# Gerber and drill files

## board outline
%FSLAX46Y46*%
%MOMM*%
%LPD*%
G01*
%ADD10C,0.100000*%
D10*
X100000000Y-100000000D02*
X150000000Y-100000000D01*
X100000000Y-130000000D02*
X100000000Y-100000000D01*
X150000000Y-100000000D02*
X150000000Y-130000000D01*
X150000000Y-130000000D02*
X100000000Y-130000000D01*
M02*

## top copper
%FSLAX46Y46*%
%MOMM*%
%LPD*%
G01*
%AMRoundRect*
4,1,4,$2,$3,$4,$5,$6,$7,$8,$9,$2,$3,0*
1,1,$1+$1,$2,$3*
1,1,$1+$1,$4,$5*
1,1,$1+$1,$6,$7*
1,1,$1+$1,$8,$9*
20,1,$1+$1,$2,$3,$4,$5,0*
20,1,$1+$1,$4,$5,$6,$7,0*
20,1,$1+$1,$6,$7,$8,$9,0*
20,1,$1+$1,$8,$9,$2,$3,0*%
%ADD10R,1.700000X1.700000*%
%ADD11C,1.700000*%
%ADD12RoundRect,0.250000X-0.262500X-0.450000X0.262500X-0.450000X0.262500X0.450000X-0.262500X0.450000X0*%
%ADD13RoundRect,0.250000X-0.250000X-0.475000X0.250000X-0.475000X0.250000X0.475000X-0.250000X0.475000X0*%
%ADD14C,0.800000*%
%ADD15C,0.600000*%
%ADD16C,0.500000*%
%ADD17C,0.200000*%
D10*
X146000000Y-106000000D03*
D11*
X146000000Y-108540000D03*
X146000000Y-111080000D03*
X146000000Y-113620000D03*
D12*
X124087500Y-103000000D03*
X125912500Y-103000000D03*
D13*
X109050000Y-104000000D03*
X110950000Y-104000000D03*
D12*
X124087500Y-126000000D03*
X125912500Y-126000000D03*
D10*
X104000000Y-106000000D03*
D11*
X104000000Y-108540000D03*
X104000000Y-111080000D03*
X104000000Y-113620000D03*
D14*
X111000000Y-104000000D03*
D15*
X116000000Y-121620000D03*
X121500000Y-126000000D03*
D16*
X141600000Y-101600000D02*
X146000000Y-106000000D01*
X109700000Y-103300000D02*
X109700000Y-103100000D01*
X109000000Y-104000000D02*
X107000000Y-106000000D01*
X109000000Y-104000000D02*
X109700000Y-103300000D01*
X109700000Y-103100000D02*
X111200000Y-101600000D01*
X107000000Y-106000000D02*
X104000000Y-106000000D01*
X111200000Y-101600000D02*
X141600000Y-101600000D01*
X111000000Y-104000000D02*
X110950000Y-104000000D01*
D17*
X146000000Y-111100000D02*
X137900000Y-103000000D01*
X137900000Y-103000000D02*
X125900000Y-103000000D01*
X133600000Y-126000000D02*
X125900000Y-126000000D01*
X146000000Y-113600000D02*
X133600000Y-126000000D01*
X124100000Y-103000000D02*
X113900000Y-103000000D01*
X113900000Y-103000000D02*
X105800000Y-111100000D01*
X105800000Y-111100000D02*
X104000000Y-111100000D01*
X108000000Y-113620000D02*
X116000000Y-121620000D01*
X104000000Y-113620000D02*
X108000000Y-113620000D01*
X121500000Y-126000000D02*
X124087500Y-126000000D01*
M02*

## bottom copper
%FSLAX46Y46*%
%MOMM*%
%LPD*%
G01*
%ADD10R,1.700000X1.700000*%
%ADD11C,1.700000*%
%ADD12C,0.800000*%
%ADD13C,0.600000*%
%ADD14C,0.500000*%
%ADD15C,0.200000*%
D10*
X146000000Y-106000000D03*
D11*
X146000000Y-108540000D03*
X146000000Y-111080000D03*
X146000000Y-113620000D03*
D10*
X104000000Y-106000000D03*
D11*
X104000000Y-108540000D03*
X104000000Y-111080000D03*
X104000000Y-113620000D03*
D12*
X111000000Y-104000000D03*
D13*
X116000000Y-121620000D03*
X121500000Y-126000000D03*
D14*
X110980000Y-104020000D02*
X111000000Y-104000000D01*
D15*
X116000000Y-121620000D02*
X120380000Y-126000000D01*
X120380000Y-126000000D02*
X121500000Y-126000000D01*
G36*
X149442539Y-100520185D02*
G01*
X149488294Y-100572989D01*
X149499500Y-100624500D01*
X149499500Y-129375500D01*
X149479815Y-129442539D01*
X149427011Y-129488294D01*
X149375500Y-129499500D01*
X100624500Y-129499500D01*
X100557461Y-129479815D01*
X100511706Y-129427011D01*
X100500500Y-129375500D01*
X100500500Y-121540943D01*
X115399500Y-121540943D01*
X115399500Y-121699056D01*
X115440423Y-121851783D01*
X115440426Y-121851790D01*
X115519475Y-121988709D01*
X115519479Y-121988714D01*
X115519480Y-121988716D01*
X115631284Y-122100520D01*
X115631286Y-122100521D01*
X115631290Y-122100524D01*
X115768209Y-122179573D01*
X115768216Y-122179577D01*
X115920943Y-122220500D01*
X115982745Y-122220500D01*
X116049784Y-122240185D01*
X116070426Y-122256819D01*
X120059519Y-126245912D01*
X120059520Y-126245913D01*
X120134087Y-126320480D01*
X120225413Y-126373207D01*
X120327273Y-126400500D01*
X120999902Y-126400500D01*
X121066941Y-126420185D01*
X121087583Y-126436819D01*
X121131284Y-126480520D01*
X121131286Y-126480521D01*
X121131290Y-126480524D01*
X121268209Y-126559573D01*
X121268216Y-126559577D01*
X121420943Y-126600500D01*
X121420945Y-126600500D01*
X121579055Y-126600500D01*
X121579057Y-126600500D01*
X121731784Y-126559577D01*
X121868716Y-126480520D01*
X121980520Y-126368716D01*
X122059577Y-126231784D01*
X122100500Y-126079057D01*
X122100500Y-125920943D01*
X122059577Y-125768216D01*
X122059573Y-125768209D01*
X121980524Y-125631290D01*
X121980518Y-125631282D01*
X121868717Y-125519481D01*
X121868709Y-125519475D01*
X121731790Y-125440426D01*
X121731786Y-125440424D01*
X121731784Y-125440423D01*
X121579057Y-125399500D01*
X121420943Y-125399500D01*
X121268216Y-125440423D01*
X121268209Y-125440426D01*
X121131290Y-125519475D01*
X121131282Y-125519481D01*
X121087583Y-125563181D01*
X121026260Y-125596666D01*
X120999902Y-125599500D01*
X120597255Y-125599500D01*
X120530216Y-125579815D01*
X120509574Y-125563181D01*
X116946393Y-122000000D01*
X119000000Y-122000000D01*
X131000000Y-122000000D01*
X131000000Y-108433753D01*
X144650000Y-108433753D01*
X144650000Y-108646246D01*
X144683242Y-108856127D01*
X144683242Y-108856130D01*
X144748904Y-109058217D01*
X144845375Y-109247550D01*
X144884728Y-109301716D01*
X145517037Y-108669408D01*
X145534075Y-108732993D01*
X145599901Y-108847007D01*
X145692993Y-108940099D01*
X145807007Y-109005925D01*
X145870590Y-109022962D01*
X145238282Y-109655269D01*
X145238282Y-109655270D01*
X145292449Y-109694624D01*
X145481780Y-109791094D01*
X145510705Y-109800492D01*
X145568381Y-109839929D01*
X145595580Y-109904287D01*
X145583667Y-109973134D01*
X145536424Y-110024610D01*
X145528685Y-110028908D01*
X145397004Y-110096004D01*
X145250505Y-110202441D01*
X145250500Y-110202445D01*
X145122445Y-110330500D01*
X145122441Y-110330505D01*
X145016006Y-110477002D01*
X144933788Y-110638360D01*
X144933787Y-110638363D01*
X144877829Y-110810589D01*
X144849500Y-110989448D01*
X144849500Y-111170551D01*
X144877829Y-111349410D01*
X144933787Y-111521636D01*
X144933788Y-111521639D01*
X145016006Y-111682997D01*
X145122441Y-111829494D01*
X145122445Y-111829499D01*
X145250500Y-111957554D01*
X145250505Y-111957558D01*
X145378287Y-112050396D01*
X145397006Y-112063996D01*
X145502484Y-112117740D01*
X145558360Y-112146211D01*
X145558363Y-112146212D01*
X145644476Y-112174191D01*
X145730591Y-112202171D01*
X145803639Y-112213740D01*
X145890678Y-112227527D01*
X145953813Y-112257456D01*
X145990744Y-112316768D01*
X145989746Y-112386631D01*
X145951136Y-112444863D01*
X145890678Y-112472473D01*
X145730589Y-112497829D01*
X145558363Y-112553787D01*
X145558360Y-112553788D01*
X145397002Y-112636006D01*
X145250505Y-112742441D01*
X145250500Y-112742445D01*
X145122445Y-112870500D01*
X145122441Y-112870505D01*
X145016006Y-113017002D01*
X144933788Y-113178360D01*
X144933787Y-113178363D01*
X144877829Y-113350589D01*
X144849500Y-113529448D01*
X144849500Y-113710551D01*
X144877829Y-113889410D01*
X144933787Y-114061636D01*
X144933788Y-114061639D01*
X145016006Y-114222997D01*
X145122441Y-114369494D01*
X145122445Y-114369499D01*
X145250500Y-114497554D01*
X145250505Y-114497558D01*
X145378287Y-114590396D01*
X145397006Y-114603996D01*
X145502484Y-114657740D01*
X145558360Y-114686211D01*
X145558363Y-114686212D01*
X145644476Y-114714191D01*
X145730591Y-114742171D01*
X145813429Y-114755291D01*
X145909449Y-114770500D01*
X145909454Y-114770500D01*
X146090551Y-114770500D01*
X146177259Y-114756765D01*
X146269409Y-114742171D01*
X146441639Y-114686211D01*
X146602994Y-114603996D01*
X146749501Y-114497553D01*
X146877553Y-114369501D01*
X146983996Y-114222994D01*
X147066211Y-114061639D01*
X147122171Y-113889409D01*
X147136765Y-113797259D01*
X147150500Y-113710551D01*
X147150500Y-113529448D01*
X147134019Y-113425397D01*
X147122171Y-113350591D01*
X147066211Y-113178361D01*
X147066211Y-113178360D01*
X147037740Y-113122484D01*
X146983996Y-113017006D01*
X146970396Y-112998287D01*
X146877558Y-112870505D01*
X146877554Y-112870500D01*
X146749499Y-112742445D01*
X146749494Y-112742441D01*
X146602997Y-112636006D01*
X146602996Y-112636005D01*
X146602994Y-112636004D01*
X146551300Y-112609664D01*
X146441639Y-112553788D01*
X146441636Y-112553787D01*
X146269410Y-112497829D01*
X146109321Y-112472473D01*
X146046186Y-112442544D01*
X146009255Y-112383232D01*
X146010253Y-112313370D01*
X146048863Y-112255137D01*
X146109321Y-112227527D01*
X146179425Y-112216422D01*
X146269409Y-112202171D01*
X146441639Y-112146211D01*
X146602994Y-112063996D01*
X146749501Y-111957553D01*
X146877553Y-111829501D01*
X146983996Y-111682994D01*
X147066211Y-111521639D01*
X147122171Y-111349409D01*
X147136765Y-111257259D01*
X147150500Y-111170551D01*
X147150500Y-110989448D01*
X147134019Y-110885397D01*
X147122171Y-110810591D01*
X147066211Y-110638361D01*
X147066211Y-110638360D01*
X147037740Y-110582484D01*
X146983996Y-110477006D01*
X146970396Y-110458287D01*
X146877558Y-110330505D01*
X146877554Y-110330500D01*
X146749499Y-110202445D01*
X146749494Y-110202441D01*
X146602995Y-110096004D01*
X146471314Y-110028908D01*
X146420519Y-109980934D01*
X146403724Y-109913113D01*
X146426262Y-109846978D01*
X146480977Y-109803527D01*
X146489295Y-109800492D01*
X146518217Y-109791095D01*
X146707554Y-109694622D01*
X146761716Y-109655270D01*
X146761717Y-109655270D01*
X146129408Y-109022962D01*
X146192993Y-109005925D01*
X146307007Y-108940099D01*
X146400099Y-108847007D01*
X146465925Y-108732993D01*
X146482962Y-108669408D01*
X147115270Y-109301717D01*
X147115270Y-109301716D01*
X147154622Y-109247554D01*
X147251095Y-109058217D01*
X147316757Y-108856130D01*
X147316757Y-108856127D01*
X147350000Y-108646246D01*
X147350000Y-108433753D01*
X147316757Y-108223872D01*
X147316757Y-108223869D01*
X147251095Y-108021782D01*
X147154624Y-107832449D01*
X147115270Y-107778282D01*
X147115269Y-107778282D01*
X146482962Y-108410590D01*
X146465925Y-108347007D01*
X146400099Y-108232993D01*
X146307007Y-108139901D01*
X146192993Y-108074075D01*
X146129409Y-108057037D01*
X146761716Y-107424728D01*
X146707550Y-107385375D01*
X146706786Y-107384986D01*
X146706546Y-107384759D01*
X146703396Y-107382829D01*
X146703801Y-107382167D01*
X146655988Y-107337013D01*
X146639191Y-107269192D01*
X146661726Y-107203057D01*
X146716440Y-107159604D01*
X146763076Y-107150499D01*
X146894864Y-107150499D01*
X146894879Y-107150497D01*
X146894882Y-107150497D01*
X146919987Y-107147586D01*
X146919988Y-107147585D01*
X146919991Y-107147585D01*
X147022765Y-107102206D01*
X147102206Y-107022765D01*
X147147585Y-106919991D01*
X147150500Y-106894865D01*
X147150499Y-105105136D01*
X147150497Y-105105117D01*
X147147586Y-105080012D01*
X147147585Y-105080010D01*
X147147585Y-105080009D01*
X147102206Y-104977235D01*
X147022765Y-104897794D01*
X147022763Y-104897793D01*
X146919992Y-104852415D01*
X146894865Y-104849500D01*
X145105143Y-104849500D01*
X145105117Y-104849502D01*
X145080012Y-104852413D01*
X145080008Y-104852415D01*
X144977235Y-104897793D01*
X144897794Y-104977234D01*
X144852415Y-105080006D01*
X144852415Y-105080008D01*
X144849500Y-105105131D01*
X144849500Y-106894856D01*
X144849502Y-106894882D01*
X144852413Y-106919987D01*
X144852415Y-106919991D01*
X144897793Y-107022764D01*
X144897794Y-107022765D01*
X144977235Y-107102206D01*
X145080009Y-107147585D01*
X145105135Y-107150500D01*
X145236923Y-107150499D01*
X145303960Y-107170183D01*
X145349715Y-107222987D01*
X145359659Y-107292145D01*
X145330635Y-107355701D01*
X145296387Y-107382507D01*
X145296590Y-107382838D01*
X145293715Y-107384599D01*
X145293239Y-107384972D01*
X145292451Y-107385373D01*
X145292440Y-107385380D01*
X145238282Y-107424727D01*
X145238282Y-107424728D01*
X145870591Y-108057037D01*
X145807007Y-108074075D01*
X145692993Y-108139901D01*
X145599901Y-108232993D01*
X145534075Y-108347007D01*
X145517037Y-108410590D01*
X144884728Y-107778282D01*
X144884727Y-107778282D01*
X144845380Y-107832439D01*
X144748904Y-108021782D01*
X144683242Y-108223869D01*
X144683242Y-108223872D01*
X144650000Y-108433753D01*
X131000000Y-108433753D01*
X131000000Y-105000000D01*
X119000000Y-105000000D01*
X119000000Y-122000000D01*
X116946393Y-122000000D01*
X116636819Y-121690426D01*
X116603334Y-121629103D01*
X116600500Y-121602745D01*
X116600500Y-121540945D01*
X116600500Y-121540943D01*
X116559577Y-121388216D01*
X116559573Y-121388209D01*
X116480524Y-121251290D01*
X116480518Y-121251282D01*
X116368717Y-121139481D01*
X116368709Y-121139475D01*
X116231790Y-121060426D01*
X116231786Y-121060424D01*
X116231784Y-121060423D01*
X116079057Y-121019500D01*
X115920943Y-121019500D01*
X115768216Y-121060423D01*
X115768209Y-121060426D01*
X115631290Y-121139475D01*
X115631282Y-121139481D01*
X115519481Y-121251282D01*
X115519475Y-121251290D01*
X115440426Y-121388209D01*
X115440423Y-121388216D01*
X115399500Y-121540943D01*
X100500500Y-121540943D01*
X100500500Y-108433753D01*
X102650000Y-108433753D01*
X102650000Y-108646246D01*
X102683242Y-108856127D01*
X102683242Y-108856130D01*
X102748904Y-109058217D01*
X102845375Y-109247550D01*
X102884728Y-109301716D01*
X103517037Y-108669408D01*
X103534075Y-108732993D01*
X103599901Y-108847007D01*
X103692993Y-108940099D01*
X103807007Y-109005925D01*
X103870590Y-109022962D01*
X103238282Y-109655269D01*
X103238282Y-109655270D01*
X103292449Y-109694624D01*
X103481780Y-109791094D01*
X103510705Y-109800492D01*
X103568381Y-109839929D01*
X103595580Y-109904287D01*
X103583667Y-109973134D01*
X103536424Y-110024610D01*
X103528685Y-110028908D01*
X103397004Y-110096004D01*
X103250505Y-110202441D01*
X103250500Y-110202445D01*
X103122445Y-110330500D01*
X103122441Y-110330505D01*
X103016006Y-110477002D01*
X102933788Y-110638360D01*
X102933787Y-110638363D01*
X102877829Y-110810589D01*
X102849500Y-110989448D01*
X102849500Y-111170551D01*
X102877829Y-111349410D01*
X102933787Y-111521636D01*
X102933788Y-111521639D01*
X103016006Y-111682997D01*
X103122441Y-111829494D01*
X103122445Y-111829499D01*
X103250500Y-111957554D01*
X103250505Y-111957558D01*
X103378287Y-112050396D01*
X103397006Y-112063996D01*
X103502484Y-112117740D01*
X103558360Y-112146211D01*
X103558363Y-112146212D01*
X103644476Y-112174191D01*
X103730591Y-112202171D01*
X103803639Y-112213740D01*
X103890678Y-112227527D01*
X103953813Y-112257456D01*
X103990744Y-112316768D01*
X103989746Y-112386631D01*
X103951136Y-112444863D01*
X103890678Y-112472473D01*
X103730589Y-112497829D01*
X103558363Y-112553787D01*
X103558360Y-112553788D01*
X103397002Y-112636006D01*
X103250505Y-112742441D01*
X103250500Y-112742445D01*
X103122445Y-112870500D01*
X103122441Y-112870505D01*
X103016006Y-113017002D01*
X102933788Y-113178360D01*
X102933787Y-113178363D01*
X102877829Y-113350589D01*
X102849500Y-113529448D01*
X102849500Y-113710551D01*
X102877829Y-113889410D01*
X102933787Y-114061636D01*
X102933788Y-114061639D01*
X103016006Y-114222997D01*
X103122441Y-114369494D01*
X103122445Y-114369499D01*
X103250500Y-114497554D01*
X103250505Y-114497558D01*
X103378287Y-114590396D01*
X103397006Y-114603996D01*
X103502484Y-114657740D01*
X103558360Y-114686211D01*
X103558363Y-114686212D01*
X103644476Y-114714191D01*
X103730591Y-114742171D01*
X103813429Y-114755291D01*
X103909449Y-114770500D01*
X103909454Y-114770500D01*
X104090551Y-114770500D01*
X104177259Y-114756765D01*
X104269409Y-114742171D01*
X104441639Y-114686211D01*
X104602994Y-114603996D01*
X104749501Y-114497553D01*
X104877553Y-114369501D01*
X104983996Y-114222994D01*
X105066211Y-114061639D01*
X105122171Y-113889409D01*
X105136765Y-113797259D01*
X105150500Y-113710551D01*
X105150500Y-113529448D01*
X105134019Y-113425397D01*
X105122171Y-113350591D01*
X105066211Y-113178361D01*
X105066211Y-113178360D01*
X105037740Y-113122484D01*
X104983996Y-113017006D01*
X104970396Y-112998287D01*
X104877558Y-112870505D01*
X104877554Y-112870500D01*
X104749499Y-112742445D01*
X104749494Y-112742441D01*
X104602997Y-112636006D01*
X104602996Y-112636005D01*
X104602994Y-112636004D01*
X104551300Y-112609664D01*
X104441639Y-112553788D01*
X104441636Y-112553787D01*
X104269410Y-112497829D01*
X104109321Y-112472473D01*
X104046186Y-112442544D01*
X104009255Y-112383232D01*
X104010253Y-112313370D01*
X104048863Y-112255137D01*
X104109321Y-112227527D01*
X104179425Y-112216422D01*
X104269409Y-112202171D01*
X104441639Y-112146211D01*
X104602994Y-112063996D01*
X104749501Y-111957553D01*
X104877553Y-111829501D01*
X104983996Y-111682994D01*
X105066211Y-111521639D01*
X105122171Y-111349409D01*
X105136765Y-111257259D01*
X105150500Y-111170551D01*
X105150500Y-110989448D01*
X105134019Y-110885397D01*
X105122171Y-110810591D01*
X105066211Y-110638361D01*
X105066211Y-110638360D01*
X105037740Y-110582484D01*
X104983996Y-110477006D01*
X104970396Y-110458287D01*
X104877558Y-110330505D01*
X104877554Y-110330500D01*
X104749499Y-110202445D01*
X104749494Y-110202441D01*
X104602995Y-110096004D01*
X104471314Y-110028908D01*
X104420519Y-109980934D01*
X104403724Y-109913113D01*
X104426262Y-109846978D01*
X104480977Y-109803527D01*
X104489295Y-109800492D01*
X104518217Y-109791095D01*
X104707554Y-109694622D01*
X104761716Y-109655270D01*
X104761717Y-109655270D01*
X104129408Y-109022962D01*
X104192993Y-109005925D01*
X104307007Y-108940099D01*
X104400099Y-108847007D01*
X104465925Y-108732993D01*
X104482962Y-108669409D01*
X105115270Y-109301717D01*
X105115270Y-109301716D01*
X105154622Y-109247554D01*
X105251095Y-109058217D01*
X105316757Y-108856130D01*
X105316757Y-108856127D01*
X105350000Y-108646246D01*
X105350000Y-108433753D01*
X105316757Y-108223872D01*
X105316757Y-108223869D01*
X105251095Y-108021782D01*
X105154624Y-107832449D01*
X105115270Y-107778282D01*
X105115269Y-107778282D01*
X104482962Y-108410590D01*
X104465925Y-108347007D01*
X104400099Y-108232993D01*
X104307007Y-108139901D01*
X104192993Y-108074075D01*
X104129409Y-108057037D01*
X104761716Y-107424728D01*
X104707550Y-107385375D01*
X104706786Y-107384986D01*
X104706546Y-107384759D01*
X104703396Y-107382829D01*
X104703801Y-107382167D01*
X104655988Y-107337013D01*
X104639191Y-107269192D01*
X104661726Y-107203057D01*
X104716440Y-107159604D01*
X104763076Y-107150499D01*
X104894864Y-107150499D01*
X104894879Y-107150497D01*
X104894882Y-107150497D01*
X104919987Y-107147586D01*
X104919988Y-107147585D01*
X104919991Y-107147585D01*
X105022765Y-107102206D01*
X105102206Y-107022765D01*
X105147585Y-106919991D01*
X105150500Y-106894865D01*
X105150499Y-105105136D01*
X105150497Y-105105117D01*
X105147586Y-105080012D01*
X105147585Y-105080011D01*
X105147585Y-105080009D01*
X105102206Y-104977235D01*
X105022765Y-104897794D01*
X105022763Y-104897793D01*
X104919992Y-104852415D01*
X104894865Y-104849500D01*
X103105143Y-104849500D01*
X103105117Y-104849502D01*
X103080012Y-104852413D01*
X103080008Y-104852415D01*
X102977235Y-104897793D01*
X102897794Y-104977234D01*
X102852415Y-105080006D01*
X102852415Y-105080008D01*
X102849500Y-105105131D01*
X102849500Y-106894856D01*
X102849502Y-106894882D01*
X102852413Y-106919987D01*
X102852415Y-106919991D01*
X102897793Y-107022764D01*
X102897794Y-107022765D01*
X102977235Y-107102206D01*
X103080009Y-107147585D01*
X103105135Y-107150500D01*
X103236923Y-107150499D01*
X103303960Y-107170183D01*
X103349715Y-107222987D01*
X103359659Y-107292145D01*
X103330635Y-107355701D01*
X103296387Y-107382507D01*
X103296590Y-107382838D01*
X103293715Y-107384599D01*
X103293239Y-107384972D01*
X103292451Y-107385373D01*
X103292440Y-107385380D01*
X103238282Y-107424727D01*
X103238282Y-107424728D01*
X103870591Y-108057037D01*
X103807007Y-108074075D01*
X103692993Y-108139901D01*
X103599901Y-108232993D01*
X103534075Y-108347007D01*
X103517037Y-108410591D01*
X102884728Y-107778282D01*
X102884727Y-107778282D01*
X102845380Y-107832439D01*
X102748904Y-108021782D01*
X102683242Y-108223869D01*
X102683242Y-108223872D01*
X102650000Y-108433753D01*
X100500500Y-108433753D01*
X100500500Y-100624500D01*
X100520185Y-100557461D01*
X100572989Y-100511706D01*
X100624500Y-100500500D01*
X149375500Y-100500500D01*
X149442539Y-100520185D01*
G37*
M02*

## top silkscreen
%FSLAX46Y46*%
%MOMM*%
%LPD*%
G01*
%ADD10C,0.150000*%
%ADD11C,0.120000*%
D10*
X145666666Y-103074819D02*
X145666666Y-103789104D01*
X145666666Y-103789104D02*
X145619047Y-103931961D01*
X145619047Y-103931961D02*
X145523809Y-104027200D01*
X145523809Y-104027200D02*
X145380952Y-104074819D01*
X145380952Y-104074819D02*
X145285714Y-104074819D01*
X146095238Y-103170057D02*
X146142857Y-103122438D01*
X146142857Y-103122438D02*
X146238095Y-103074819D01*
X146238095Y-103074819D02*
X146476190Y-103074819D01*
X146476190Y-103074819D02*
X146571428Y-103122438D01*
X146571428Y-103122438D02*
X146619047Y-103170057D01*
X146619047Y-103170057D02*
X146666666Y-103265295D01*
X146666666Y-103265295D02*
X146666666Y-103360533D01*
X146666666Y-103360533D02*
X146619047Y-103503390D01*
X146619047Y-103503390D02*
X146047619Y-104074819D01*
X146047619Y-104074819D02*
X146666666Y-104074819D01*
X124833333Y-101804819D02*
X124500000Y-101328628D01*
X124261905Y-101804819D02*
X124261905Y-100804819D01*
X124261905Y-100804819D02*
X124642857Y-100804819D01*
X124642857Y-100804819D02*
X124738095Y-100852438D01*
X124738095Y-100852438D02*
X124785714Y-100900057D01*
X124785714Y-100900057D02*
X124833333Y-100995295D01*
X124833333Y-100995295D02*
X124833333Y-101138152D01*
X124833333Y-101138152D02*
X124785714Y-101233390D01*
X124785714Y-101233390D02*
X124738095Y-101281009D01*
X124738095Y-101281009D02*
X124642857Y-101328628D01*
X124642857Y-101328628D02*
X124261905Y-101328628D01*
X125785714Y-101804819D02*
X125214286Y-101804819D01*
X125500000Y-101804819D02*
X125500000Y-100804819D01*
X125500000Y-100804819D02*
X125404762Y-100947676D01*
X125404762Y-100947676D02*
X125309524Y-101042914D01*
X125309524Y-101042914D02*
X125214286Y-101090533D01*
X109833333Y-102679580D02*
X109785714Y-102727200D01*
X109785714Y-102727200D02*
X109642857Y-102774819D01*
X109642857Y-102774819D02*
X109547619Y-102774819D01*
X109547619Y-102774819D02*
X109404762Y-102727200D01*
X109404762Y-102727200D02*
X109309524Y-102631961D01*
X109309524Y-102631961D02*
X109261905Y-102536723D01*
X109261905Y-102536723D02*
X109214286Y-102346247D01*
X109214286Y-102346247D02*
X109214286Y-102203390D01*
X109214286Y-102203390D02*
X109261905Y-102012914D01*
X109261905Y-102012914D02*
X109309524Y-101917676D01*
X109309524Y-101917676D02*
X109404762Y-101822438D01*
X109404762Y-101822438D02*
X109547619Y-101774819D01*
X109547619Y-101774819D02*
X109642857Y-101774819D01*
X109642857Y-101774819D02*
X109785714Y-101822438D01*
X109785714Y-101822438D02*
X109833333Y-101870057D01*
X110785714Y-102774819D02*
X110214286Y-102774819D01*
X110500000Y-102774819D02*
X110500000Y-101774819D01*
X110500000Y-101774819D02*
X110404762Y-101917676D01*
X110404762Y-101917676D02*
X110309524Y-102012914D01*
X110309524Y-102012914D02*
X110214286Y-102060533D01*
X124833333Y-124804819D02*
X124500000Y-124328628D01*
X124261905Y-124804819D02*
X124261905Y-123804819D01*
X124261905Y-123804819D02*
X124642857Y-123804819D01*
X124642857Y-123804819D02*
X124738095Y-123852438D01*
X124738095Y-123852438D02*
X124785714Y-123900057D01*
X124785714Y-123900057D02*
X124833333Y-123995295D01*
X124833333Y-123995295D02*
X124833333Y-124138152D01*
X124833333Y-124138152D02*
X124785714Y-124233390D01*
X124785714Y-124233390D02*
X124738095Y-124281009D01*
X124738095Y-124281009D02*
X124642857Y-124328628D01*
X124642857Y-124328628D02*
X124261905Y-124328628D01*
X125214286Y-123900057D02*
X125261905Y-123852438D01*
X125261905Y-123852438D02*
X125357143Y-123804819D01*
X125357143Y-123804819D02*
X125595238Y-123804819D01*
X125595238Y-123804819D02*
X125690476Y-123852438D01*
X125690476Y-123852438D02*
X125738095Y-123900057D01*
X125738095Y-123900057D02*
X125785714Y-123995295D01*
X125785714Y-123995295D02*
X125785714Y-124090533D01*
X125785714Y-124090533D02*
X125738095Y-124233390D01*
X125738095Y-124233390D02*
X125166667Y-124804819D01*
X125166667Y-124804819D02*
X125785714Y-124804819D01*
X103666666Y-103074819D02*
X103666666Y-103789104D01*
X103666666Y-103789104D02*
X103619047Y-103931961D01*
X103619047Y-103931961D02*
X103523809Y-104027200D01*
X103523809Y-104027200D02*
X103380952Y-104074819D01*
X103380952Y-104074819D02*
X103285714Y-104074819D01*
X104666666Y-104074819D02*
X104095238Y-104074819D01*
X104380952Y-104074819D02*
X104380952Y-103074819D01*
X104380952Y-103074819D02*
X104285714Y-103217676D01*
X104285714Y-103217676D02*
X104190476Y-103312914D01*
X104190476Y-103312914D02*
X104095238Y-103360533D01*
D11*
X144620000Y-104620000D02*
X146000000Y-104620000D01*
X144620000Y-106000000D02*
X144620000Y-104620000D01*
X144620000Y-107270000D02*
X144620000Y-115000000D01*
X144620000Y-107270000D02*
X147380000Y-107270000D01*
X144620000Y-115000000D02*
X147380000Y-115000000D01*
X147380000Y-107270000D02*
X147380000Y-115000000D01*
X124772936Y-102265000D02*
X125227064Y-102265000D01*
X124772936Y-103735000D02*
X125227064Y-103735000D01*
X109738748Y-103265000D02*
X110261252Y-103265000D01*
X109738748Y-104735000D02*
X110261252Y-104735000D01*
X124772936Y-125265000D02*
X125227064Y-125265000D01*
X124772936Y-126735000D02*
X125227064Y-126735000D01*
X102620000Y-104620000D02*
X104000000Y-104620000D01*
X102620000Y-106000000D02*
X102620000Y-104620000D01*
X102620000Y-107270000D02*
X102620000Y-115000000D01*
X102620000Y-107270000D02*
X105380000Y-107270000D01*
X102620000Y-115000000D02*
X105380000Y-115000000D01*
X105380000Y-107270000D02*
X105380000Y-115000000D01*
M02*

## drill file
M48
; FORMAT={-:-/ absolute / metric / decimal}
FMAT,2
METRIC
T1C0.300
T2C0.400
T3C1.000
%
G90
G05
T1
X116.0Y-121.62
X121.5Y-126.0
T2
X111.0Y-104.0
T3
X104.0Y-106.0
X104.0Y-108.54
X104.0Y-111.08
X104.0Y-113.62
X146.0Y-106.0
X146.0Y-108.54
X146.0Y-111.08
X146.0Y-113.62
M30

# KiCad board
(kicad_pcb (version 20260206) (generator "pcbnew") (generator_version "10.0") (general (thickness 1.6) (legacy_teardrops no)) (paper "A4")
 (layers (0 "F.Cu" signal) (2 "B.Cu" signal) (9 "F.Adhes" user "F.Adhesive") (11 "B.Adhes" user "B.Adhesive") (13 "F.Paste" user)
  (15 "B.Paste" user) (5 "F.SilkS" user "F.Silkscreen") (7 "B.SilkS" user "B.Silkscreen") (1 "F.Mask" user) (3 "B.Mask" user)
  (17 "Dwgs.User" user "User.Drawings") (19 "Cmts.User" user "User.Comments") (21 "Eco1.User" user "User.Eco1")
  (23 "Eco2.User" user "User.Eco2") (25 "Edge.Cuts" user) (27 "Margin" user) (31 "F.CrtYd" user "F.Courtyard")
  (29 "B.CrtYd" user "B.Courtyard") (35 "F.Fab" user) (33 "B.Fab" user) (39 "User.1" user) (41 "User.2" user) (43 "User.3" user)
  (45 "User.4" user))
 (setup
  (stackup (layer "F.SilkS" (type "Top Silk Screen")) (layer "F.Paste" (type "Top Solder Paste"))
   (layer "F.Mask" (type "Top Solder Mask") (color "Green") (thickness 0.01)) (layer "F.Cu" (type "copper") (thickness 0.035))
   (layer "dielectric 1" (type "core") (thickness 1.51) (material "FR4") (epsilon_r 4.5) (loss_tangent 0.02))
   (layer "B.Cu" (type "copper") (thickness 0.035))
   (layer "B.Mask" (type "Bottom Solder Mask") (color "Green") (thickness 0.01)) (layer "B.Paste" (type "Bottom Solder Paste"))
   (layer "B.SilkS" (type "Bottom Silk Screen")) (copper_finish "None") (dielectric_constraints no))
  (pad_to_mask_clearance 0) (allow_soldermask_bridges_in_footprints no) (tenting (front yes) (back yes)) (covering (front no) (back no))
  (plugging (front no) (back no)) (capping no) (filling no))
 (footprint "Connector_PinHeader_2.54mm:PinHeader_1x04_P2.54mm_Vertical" (layer "F.Cu") (at 146 106)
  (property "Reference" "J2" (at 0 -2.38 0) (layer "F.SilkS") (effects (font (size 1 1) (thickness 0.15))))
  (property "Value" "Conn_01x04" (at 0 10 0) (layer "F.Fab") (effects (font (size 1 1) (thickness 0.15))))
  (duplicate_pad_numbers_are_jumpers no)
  (fp_line (start -1.38 -1.38) (end 0 -1.38) (stroke (width 0.12) (type solid)) (layer "F.SilkS"))
  (fp_line (start -1.38 0) (end -1.38 -1.38) (stroke (width 0.12) (type solid)) (layer "F.SilkS"))
  (fp_line (start -1.38 1.27) (end -1.38 9) (stroke (width 0.12) (type solid)) (layer "F.SilkS"))
  (fp_line (start -1.38 1.27) (end 1.38 1.27) (stroke (width 0.12) (type solid)) (layer "F.SilkS"))
  (fp_line (start -1.38 9) (end 1.38 9) (stroke (width 0.12) (type solid)) (layer "F.SilkS"))
  (fp_line (start 1.38 1.27) (end 1.38 9) (stroke (width 0.12) (type solid)) (layer "F.SilkS"))
  (pad "1" thru_hole rect (at 0 0) (size 1.7 1.7) (drill 1) (layers "*.Cu" "*.Mask") (remove_unused_layers no) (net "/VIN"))
  (pad "2" thru_hole circle (at 0 2.54) (size 1.7 1.7) (drill 1) (layers "*.Cu" "*.Mask") (remove_unused_layers no) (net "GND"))
  (pad "3" thru_hole circle (at 0 5.08) (size 1.7 1.7) (drill 1) (layers "*.Cu" "*.Mask") (remove_unused_layers no) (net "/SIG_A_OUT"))
  (pad "4" thru_hole circle (at 0 7.62) (size 1.7 1.7) (drill 1) (layers "*.Cu" "*.Mask") (remove_unused_layers no) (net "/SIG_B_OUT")))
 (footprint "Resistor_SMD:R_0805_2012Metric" (layer "F.Cu") (at 125 103)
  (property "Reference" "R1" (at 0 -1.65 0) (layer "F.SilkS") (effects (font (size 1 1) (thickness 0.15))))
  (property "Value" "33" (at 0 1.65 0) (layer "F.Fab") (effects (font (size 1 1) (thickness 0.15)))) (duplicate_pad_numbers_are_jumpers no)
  (fp_line (start -0.227064 -0.735) (end 0.227064 -0.735) (stroke (width 0.12) (type solid)) (layer "F.SilkS"))
  (fp_line (start -0.227064 0.735) (end 0.227064 0.735) (stroke (width 0.12) (type solid)) (layer "F.SilkS"))
  (pad "1" smd roundrect (at -0.9125 0) (size 1.025 1.4) (layers "F.Cu" "F.Mask" "F.Paste") (roundrect_rratio 0.243902) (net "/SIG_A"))
  (pad "2" smd roundrect (at 0.9125 0) (size 1.025 1.4) (layers "F.Cu" "F.Mask" "F.Paste") (roundrect_rratio 0.243902) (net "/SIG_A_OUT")))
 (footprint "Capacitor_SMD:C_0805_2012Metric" (layer "F.Cu") (at 110 104)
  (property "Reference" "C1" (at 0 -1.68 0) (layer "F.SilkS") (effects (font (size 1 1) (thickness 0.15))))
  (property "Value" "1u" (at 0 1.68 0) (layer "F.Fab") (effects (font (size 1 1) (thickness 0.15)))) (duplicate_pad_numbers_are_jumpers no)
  (fp_line (start -0.261252 -0.735) (end 0.261252 -0.735) (stroke (width 0.12) (type solid)) (layer "F.SilkS"))
  (fp_line (start -0.261252 0.735) (end 0.261252 0.735) (stroke (width 0.12) (type solid)) (layer "F.SilkS"))
  (pad "1" smd roundrect (at -0.95 0) (size 1 1.45) (layers "F.Cu" "F.Mask" "F.Paste") (roundrect_rratio 0.25) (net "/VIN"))
  (pad "2" smd roundrect (at 0.95 0) (size 1 1.45) (layers "F.Cu" "F.Mask" "F.Paste") (roundrect_rratio 0.25) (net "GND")))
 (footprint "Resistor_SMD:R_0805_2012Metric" (layer "F.Cu") (at 125 126)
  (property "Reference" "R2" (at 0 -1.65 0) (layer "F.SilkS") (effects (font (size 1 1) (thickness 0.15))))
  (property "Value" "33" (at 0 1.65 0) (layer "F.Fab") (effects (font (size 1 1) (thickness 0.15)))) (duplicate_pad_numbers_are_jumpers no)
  (fp_line (start -0.227064 -0.735) (end 0.227064 -0.735) (stroke (width 0.12) (type solid)) (layer "F.SilkS"))
  (fp_line (start -0.227064 0.735) (end 0.227064 0.735) (stroke (width 0.12) (type solid)) (layer "F.SilkS"))
  (pad "1" smd roundrect (at -0.9125 0) (size 1.025 1.4) (layers "F.Cu" "F.Mask" "F.Paste") (roundrect_rratio 0.243902) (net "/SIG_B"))
  (pad "2" smd roundrect (at 0.9125 0) (size 1.025 1.4) (layers "F.Cu" "F.Mask" "F.Paste") (roundrect_rratio 0.243902) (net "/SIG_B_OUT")))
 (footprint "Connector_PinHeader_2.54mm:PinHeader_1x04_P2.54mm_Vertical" (layer "F.Cu") (at 104 106)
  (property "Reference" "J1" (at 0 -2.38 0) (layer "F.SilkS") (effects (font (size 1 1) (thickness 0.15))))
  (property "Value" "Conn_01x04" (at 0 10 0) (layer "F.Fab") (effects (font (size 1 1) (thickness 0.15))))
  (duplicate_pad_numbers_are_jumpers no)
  (fp_line (start -1.38 -1.38) (end 0 -1.38) (stroke (width 0.12) (type solid)) (layer "F.SilkS"))
  (fp_line (start -1.38 0) (end -1.38 -1.38) (stroke (width 0.12) (type solid)) (layer "F.SilkS"))
  (fp_line (start -1.38 1.27) (end -1.38 9) (stroke (width 0.12) (type solid)) (layer "F.SilkS"))
  (fp_line (start -1.38 1.27) (end 1.38 1.27) (stroke (width 0.12) (type solid)) (layer "F.SilkS"))
  (fp_line (start -1.38 9) (end 1.38 9) (stroke (width 0.12) (type solid)) (layer "F.SilkS"))
  (fp_line (start 1.38 1.27) (end 1.38 9) (stroke (width 0.12) (type solid)) (layer "F.SilkS"))
  (pad "1" thru_hole rect (at 0 0) (size 1.7 1.7) (drill 1) (layers "*.Cu" "*.Mask") (remove_unused_layers no) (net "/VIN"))
  (pad "2" thru_hole circle (at 0 2.54) (size 1.7 1.7) (drill 1) (layers "*.Cu" "*.Mask") (remove_unused_layers no) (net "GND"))
  (pad "3" thru_hole circle (at 0 5.08) (size 1.7 1.7) (drill 1) (layers "*.Cu" "*.Mask") (remove_unused_layers no) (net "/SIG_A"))
  (pad "4" thru_hole circle (at 0 7.62) (size 1.7 1.7) (drill 1) (layers "*.Cu" "*.Mask") (remove_unused_layers no) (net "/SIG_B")))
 (gr_line (start 100 100) (end 150 100) (stroke (width 0.1) (type default)) (layer "Edge.Cuts"))
 (gr_line (start 100 130) (end 100 100) (stroke (width 0.1) (type default)) (layer "Edge.Cuts"))
 (gr_line (start 150 100) (end 150 130) (stroke (width 0.1) (type default)) (layer "Edge.Cuts"))
 (gr_line (start 150 130) (end 100 130) (stroke (width 0.1) (type default)) (layer "Edge.Cuts"))
 (segment (start 141.6 101.6) (end 146 106) (width 0.5) (layer "F.Cu") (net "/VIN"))
 (segment (start 109.7 103.3) (end 109.7 103.1) (width 0.5) (layer "F.Cu") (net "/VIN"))
 (segment (start 109 104) (end 107 106) (width 0.5) (layer "F.Cu") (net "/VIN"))
 (segment (start 109 104) (end 109.7 103.3) (width 0.5) (layer "F.Cu") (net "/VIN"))
 (segment (start 109.7 103.1) (end 111.2 101.6) (width 0.5) (layer "F.Cu") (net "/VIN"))
 (segment (start 107 106) (end 104 106) (width 0.5) (layer "F.Cu") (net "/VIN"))
 (segment (start 111.2 101.6) (end 141.6 101.6) (width 0.5) (layer "F.Cu") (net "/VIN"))
 (segment (start 111 104) (end 110.95 104) (width 0.5) (layer "F.Cu") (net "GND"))
 (via (at 111 104) (size 0.8) (drill 0.4) (layers "F.Cu" "B.Cu") (capping yes) (filling yes) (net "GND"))
 (segment (start 110.98 104.02) (end 111 104) (width 0.5) (layer "B.Cu") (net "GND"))
 (segment (start 146 111.1) (end 137.9 103) (width 0.2) (layer "F.Cu") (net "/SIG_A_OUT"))
 (segment (start 137.9 103) (end 125.9 103) (width 0.2) (layer "F.Cu") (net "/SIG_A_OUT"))
 (segment (start 133.6 126) (end 125.9 126) (width 0.2) (layer "F.Cu") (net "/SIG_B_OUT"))
 (segment (start 146 113.6) (end 133.6 126) (width 0.2) (layer "F.Cu") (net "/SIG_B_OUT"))
 (segment (start 124.1 103) (end 113.9 103) (width 0.2) (layer "F.Cu") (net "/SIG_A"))
 (segment (start 113.9 103) (end 105.8 111.1) (width 0.2) (layer "F.Cu") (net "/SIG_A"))
 (segment (start 105.8 111.1) (end 104 111.1) (width 0.2) (layer "F.Cu") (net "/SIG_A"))
 (segment (start 108 113.62) (end 116 121.62) (width 0.2) (locked yes) (layer "F.Cu") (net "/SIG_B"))
 (segment (start 104 113.62) (end 108 113.62) (width 0.2) (locked yes) (layer "F.Cu") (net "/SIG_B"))
 (segment (start 121.5 126) (end 124.0875 126) (width 0.2) (locked yes) (layer "F.Cu") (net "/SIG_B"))
 (via (at 116 121.62) (size 0.6) (drill 0.3) (layers "F.Cu" "B.Cu") (locked yes) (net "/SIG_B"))
 (via (at 121.5 126) (size 0.6) (drill 0.3) (layers "F.Cu" "B.Cu") (locked yes) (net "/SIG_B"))
 (segment (start 116 121.62) (end 120.38 126) (width 0.2) (locked yes) (layer "B.Cu") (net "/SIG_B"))
 (segment (start 120.38 126) (end 121.5 126) (width 0.2) (locked yes) (layer "B.Cu") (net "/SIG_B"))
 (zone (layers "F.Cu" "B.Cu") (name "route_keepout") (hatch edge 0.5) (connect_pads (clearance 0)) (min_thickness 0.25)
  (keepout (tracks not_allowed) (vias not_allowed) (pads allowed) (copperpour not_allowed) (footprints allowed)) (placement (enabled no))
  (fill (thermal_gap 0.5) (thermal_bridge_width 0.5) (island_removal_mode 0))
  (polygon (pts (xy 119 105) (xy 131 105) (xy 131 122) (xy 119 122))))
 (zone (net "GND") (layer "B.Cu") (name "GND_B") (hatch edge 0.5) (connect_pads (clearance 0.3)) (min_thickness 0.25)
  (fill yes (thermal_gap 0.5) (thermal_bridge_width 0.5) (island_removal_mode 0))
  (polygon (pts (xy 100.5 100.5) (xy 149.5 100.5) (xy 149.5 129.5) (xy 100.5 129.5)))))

